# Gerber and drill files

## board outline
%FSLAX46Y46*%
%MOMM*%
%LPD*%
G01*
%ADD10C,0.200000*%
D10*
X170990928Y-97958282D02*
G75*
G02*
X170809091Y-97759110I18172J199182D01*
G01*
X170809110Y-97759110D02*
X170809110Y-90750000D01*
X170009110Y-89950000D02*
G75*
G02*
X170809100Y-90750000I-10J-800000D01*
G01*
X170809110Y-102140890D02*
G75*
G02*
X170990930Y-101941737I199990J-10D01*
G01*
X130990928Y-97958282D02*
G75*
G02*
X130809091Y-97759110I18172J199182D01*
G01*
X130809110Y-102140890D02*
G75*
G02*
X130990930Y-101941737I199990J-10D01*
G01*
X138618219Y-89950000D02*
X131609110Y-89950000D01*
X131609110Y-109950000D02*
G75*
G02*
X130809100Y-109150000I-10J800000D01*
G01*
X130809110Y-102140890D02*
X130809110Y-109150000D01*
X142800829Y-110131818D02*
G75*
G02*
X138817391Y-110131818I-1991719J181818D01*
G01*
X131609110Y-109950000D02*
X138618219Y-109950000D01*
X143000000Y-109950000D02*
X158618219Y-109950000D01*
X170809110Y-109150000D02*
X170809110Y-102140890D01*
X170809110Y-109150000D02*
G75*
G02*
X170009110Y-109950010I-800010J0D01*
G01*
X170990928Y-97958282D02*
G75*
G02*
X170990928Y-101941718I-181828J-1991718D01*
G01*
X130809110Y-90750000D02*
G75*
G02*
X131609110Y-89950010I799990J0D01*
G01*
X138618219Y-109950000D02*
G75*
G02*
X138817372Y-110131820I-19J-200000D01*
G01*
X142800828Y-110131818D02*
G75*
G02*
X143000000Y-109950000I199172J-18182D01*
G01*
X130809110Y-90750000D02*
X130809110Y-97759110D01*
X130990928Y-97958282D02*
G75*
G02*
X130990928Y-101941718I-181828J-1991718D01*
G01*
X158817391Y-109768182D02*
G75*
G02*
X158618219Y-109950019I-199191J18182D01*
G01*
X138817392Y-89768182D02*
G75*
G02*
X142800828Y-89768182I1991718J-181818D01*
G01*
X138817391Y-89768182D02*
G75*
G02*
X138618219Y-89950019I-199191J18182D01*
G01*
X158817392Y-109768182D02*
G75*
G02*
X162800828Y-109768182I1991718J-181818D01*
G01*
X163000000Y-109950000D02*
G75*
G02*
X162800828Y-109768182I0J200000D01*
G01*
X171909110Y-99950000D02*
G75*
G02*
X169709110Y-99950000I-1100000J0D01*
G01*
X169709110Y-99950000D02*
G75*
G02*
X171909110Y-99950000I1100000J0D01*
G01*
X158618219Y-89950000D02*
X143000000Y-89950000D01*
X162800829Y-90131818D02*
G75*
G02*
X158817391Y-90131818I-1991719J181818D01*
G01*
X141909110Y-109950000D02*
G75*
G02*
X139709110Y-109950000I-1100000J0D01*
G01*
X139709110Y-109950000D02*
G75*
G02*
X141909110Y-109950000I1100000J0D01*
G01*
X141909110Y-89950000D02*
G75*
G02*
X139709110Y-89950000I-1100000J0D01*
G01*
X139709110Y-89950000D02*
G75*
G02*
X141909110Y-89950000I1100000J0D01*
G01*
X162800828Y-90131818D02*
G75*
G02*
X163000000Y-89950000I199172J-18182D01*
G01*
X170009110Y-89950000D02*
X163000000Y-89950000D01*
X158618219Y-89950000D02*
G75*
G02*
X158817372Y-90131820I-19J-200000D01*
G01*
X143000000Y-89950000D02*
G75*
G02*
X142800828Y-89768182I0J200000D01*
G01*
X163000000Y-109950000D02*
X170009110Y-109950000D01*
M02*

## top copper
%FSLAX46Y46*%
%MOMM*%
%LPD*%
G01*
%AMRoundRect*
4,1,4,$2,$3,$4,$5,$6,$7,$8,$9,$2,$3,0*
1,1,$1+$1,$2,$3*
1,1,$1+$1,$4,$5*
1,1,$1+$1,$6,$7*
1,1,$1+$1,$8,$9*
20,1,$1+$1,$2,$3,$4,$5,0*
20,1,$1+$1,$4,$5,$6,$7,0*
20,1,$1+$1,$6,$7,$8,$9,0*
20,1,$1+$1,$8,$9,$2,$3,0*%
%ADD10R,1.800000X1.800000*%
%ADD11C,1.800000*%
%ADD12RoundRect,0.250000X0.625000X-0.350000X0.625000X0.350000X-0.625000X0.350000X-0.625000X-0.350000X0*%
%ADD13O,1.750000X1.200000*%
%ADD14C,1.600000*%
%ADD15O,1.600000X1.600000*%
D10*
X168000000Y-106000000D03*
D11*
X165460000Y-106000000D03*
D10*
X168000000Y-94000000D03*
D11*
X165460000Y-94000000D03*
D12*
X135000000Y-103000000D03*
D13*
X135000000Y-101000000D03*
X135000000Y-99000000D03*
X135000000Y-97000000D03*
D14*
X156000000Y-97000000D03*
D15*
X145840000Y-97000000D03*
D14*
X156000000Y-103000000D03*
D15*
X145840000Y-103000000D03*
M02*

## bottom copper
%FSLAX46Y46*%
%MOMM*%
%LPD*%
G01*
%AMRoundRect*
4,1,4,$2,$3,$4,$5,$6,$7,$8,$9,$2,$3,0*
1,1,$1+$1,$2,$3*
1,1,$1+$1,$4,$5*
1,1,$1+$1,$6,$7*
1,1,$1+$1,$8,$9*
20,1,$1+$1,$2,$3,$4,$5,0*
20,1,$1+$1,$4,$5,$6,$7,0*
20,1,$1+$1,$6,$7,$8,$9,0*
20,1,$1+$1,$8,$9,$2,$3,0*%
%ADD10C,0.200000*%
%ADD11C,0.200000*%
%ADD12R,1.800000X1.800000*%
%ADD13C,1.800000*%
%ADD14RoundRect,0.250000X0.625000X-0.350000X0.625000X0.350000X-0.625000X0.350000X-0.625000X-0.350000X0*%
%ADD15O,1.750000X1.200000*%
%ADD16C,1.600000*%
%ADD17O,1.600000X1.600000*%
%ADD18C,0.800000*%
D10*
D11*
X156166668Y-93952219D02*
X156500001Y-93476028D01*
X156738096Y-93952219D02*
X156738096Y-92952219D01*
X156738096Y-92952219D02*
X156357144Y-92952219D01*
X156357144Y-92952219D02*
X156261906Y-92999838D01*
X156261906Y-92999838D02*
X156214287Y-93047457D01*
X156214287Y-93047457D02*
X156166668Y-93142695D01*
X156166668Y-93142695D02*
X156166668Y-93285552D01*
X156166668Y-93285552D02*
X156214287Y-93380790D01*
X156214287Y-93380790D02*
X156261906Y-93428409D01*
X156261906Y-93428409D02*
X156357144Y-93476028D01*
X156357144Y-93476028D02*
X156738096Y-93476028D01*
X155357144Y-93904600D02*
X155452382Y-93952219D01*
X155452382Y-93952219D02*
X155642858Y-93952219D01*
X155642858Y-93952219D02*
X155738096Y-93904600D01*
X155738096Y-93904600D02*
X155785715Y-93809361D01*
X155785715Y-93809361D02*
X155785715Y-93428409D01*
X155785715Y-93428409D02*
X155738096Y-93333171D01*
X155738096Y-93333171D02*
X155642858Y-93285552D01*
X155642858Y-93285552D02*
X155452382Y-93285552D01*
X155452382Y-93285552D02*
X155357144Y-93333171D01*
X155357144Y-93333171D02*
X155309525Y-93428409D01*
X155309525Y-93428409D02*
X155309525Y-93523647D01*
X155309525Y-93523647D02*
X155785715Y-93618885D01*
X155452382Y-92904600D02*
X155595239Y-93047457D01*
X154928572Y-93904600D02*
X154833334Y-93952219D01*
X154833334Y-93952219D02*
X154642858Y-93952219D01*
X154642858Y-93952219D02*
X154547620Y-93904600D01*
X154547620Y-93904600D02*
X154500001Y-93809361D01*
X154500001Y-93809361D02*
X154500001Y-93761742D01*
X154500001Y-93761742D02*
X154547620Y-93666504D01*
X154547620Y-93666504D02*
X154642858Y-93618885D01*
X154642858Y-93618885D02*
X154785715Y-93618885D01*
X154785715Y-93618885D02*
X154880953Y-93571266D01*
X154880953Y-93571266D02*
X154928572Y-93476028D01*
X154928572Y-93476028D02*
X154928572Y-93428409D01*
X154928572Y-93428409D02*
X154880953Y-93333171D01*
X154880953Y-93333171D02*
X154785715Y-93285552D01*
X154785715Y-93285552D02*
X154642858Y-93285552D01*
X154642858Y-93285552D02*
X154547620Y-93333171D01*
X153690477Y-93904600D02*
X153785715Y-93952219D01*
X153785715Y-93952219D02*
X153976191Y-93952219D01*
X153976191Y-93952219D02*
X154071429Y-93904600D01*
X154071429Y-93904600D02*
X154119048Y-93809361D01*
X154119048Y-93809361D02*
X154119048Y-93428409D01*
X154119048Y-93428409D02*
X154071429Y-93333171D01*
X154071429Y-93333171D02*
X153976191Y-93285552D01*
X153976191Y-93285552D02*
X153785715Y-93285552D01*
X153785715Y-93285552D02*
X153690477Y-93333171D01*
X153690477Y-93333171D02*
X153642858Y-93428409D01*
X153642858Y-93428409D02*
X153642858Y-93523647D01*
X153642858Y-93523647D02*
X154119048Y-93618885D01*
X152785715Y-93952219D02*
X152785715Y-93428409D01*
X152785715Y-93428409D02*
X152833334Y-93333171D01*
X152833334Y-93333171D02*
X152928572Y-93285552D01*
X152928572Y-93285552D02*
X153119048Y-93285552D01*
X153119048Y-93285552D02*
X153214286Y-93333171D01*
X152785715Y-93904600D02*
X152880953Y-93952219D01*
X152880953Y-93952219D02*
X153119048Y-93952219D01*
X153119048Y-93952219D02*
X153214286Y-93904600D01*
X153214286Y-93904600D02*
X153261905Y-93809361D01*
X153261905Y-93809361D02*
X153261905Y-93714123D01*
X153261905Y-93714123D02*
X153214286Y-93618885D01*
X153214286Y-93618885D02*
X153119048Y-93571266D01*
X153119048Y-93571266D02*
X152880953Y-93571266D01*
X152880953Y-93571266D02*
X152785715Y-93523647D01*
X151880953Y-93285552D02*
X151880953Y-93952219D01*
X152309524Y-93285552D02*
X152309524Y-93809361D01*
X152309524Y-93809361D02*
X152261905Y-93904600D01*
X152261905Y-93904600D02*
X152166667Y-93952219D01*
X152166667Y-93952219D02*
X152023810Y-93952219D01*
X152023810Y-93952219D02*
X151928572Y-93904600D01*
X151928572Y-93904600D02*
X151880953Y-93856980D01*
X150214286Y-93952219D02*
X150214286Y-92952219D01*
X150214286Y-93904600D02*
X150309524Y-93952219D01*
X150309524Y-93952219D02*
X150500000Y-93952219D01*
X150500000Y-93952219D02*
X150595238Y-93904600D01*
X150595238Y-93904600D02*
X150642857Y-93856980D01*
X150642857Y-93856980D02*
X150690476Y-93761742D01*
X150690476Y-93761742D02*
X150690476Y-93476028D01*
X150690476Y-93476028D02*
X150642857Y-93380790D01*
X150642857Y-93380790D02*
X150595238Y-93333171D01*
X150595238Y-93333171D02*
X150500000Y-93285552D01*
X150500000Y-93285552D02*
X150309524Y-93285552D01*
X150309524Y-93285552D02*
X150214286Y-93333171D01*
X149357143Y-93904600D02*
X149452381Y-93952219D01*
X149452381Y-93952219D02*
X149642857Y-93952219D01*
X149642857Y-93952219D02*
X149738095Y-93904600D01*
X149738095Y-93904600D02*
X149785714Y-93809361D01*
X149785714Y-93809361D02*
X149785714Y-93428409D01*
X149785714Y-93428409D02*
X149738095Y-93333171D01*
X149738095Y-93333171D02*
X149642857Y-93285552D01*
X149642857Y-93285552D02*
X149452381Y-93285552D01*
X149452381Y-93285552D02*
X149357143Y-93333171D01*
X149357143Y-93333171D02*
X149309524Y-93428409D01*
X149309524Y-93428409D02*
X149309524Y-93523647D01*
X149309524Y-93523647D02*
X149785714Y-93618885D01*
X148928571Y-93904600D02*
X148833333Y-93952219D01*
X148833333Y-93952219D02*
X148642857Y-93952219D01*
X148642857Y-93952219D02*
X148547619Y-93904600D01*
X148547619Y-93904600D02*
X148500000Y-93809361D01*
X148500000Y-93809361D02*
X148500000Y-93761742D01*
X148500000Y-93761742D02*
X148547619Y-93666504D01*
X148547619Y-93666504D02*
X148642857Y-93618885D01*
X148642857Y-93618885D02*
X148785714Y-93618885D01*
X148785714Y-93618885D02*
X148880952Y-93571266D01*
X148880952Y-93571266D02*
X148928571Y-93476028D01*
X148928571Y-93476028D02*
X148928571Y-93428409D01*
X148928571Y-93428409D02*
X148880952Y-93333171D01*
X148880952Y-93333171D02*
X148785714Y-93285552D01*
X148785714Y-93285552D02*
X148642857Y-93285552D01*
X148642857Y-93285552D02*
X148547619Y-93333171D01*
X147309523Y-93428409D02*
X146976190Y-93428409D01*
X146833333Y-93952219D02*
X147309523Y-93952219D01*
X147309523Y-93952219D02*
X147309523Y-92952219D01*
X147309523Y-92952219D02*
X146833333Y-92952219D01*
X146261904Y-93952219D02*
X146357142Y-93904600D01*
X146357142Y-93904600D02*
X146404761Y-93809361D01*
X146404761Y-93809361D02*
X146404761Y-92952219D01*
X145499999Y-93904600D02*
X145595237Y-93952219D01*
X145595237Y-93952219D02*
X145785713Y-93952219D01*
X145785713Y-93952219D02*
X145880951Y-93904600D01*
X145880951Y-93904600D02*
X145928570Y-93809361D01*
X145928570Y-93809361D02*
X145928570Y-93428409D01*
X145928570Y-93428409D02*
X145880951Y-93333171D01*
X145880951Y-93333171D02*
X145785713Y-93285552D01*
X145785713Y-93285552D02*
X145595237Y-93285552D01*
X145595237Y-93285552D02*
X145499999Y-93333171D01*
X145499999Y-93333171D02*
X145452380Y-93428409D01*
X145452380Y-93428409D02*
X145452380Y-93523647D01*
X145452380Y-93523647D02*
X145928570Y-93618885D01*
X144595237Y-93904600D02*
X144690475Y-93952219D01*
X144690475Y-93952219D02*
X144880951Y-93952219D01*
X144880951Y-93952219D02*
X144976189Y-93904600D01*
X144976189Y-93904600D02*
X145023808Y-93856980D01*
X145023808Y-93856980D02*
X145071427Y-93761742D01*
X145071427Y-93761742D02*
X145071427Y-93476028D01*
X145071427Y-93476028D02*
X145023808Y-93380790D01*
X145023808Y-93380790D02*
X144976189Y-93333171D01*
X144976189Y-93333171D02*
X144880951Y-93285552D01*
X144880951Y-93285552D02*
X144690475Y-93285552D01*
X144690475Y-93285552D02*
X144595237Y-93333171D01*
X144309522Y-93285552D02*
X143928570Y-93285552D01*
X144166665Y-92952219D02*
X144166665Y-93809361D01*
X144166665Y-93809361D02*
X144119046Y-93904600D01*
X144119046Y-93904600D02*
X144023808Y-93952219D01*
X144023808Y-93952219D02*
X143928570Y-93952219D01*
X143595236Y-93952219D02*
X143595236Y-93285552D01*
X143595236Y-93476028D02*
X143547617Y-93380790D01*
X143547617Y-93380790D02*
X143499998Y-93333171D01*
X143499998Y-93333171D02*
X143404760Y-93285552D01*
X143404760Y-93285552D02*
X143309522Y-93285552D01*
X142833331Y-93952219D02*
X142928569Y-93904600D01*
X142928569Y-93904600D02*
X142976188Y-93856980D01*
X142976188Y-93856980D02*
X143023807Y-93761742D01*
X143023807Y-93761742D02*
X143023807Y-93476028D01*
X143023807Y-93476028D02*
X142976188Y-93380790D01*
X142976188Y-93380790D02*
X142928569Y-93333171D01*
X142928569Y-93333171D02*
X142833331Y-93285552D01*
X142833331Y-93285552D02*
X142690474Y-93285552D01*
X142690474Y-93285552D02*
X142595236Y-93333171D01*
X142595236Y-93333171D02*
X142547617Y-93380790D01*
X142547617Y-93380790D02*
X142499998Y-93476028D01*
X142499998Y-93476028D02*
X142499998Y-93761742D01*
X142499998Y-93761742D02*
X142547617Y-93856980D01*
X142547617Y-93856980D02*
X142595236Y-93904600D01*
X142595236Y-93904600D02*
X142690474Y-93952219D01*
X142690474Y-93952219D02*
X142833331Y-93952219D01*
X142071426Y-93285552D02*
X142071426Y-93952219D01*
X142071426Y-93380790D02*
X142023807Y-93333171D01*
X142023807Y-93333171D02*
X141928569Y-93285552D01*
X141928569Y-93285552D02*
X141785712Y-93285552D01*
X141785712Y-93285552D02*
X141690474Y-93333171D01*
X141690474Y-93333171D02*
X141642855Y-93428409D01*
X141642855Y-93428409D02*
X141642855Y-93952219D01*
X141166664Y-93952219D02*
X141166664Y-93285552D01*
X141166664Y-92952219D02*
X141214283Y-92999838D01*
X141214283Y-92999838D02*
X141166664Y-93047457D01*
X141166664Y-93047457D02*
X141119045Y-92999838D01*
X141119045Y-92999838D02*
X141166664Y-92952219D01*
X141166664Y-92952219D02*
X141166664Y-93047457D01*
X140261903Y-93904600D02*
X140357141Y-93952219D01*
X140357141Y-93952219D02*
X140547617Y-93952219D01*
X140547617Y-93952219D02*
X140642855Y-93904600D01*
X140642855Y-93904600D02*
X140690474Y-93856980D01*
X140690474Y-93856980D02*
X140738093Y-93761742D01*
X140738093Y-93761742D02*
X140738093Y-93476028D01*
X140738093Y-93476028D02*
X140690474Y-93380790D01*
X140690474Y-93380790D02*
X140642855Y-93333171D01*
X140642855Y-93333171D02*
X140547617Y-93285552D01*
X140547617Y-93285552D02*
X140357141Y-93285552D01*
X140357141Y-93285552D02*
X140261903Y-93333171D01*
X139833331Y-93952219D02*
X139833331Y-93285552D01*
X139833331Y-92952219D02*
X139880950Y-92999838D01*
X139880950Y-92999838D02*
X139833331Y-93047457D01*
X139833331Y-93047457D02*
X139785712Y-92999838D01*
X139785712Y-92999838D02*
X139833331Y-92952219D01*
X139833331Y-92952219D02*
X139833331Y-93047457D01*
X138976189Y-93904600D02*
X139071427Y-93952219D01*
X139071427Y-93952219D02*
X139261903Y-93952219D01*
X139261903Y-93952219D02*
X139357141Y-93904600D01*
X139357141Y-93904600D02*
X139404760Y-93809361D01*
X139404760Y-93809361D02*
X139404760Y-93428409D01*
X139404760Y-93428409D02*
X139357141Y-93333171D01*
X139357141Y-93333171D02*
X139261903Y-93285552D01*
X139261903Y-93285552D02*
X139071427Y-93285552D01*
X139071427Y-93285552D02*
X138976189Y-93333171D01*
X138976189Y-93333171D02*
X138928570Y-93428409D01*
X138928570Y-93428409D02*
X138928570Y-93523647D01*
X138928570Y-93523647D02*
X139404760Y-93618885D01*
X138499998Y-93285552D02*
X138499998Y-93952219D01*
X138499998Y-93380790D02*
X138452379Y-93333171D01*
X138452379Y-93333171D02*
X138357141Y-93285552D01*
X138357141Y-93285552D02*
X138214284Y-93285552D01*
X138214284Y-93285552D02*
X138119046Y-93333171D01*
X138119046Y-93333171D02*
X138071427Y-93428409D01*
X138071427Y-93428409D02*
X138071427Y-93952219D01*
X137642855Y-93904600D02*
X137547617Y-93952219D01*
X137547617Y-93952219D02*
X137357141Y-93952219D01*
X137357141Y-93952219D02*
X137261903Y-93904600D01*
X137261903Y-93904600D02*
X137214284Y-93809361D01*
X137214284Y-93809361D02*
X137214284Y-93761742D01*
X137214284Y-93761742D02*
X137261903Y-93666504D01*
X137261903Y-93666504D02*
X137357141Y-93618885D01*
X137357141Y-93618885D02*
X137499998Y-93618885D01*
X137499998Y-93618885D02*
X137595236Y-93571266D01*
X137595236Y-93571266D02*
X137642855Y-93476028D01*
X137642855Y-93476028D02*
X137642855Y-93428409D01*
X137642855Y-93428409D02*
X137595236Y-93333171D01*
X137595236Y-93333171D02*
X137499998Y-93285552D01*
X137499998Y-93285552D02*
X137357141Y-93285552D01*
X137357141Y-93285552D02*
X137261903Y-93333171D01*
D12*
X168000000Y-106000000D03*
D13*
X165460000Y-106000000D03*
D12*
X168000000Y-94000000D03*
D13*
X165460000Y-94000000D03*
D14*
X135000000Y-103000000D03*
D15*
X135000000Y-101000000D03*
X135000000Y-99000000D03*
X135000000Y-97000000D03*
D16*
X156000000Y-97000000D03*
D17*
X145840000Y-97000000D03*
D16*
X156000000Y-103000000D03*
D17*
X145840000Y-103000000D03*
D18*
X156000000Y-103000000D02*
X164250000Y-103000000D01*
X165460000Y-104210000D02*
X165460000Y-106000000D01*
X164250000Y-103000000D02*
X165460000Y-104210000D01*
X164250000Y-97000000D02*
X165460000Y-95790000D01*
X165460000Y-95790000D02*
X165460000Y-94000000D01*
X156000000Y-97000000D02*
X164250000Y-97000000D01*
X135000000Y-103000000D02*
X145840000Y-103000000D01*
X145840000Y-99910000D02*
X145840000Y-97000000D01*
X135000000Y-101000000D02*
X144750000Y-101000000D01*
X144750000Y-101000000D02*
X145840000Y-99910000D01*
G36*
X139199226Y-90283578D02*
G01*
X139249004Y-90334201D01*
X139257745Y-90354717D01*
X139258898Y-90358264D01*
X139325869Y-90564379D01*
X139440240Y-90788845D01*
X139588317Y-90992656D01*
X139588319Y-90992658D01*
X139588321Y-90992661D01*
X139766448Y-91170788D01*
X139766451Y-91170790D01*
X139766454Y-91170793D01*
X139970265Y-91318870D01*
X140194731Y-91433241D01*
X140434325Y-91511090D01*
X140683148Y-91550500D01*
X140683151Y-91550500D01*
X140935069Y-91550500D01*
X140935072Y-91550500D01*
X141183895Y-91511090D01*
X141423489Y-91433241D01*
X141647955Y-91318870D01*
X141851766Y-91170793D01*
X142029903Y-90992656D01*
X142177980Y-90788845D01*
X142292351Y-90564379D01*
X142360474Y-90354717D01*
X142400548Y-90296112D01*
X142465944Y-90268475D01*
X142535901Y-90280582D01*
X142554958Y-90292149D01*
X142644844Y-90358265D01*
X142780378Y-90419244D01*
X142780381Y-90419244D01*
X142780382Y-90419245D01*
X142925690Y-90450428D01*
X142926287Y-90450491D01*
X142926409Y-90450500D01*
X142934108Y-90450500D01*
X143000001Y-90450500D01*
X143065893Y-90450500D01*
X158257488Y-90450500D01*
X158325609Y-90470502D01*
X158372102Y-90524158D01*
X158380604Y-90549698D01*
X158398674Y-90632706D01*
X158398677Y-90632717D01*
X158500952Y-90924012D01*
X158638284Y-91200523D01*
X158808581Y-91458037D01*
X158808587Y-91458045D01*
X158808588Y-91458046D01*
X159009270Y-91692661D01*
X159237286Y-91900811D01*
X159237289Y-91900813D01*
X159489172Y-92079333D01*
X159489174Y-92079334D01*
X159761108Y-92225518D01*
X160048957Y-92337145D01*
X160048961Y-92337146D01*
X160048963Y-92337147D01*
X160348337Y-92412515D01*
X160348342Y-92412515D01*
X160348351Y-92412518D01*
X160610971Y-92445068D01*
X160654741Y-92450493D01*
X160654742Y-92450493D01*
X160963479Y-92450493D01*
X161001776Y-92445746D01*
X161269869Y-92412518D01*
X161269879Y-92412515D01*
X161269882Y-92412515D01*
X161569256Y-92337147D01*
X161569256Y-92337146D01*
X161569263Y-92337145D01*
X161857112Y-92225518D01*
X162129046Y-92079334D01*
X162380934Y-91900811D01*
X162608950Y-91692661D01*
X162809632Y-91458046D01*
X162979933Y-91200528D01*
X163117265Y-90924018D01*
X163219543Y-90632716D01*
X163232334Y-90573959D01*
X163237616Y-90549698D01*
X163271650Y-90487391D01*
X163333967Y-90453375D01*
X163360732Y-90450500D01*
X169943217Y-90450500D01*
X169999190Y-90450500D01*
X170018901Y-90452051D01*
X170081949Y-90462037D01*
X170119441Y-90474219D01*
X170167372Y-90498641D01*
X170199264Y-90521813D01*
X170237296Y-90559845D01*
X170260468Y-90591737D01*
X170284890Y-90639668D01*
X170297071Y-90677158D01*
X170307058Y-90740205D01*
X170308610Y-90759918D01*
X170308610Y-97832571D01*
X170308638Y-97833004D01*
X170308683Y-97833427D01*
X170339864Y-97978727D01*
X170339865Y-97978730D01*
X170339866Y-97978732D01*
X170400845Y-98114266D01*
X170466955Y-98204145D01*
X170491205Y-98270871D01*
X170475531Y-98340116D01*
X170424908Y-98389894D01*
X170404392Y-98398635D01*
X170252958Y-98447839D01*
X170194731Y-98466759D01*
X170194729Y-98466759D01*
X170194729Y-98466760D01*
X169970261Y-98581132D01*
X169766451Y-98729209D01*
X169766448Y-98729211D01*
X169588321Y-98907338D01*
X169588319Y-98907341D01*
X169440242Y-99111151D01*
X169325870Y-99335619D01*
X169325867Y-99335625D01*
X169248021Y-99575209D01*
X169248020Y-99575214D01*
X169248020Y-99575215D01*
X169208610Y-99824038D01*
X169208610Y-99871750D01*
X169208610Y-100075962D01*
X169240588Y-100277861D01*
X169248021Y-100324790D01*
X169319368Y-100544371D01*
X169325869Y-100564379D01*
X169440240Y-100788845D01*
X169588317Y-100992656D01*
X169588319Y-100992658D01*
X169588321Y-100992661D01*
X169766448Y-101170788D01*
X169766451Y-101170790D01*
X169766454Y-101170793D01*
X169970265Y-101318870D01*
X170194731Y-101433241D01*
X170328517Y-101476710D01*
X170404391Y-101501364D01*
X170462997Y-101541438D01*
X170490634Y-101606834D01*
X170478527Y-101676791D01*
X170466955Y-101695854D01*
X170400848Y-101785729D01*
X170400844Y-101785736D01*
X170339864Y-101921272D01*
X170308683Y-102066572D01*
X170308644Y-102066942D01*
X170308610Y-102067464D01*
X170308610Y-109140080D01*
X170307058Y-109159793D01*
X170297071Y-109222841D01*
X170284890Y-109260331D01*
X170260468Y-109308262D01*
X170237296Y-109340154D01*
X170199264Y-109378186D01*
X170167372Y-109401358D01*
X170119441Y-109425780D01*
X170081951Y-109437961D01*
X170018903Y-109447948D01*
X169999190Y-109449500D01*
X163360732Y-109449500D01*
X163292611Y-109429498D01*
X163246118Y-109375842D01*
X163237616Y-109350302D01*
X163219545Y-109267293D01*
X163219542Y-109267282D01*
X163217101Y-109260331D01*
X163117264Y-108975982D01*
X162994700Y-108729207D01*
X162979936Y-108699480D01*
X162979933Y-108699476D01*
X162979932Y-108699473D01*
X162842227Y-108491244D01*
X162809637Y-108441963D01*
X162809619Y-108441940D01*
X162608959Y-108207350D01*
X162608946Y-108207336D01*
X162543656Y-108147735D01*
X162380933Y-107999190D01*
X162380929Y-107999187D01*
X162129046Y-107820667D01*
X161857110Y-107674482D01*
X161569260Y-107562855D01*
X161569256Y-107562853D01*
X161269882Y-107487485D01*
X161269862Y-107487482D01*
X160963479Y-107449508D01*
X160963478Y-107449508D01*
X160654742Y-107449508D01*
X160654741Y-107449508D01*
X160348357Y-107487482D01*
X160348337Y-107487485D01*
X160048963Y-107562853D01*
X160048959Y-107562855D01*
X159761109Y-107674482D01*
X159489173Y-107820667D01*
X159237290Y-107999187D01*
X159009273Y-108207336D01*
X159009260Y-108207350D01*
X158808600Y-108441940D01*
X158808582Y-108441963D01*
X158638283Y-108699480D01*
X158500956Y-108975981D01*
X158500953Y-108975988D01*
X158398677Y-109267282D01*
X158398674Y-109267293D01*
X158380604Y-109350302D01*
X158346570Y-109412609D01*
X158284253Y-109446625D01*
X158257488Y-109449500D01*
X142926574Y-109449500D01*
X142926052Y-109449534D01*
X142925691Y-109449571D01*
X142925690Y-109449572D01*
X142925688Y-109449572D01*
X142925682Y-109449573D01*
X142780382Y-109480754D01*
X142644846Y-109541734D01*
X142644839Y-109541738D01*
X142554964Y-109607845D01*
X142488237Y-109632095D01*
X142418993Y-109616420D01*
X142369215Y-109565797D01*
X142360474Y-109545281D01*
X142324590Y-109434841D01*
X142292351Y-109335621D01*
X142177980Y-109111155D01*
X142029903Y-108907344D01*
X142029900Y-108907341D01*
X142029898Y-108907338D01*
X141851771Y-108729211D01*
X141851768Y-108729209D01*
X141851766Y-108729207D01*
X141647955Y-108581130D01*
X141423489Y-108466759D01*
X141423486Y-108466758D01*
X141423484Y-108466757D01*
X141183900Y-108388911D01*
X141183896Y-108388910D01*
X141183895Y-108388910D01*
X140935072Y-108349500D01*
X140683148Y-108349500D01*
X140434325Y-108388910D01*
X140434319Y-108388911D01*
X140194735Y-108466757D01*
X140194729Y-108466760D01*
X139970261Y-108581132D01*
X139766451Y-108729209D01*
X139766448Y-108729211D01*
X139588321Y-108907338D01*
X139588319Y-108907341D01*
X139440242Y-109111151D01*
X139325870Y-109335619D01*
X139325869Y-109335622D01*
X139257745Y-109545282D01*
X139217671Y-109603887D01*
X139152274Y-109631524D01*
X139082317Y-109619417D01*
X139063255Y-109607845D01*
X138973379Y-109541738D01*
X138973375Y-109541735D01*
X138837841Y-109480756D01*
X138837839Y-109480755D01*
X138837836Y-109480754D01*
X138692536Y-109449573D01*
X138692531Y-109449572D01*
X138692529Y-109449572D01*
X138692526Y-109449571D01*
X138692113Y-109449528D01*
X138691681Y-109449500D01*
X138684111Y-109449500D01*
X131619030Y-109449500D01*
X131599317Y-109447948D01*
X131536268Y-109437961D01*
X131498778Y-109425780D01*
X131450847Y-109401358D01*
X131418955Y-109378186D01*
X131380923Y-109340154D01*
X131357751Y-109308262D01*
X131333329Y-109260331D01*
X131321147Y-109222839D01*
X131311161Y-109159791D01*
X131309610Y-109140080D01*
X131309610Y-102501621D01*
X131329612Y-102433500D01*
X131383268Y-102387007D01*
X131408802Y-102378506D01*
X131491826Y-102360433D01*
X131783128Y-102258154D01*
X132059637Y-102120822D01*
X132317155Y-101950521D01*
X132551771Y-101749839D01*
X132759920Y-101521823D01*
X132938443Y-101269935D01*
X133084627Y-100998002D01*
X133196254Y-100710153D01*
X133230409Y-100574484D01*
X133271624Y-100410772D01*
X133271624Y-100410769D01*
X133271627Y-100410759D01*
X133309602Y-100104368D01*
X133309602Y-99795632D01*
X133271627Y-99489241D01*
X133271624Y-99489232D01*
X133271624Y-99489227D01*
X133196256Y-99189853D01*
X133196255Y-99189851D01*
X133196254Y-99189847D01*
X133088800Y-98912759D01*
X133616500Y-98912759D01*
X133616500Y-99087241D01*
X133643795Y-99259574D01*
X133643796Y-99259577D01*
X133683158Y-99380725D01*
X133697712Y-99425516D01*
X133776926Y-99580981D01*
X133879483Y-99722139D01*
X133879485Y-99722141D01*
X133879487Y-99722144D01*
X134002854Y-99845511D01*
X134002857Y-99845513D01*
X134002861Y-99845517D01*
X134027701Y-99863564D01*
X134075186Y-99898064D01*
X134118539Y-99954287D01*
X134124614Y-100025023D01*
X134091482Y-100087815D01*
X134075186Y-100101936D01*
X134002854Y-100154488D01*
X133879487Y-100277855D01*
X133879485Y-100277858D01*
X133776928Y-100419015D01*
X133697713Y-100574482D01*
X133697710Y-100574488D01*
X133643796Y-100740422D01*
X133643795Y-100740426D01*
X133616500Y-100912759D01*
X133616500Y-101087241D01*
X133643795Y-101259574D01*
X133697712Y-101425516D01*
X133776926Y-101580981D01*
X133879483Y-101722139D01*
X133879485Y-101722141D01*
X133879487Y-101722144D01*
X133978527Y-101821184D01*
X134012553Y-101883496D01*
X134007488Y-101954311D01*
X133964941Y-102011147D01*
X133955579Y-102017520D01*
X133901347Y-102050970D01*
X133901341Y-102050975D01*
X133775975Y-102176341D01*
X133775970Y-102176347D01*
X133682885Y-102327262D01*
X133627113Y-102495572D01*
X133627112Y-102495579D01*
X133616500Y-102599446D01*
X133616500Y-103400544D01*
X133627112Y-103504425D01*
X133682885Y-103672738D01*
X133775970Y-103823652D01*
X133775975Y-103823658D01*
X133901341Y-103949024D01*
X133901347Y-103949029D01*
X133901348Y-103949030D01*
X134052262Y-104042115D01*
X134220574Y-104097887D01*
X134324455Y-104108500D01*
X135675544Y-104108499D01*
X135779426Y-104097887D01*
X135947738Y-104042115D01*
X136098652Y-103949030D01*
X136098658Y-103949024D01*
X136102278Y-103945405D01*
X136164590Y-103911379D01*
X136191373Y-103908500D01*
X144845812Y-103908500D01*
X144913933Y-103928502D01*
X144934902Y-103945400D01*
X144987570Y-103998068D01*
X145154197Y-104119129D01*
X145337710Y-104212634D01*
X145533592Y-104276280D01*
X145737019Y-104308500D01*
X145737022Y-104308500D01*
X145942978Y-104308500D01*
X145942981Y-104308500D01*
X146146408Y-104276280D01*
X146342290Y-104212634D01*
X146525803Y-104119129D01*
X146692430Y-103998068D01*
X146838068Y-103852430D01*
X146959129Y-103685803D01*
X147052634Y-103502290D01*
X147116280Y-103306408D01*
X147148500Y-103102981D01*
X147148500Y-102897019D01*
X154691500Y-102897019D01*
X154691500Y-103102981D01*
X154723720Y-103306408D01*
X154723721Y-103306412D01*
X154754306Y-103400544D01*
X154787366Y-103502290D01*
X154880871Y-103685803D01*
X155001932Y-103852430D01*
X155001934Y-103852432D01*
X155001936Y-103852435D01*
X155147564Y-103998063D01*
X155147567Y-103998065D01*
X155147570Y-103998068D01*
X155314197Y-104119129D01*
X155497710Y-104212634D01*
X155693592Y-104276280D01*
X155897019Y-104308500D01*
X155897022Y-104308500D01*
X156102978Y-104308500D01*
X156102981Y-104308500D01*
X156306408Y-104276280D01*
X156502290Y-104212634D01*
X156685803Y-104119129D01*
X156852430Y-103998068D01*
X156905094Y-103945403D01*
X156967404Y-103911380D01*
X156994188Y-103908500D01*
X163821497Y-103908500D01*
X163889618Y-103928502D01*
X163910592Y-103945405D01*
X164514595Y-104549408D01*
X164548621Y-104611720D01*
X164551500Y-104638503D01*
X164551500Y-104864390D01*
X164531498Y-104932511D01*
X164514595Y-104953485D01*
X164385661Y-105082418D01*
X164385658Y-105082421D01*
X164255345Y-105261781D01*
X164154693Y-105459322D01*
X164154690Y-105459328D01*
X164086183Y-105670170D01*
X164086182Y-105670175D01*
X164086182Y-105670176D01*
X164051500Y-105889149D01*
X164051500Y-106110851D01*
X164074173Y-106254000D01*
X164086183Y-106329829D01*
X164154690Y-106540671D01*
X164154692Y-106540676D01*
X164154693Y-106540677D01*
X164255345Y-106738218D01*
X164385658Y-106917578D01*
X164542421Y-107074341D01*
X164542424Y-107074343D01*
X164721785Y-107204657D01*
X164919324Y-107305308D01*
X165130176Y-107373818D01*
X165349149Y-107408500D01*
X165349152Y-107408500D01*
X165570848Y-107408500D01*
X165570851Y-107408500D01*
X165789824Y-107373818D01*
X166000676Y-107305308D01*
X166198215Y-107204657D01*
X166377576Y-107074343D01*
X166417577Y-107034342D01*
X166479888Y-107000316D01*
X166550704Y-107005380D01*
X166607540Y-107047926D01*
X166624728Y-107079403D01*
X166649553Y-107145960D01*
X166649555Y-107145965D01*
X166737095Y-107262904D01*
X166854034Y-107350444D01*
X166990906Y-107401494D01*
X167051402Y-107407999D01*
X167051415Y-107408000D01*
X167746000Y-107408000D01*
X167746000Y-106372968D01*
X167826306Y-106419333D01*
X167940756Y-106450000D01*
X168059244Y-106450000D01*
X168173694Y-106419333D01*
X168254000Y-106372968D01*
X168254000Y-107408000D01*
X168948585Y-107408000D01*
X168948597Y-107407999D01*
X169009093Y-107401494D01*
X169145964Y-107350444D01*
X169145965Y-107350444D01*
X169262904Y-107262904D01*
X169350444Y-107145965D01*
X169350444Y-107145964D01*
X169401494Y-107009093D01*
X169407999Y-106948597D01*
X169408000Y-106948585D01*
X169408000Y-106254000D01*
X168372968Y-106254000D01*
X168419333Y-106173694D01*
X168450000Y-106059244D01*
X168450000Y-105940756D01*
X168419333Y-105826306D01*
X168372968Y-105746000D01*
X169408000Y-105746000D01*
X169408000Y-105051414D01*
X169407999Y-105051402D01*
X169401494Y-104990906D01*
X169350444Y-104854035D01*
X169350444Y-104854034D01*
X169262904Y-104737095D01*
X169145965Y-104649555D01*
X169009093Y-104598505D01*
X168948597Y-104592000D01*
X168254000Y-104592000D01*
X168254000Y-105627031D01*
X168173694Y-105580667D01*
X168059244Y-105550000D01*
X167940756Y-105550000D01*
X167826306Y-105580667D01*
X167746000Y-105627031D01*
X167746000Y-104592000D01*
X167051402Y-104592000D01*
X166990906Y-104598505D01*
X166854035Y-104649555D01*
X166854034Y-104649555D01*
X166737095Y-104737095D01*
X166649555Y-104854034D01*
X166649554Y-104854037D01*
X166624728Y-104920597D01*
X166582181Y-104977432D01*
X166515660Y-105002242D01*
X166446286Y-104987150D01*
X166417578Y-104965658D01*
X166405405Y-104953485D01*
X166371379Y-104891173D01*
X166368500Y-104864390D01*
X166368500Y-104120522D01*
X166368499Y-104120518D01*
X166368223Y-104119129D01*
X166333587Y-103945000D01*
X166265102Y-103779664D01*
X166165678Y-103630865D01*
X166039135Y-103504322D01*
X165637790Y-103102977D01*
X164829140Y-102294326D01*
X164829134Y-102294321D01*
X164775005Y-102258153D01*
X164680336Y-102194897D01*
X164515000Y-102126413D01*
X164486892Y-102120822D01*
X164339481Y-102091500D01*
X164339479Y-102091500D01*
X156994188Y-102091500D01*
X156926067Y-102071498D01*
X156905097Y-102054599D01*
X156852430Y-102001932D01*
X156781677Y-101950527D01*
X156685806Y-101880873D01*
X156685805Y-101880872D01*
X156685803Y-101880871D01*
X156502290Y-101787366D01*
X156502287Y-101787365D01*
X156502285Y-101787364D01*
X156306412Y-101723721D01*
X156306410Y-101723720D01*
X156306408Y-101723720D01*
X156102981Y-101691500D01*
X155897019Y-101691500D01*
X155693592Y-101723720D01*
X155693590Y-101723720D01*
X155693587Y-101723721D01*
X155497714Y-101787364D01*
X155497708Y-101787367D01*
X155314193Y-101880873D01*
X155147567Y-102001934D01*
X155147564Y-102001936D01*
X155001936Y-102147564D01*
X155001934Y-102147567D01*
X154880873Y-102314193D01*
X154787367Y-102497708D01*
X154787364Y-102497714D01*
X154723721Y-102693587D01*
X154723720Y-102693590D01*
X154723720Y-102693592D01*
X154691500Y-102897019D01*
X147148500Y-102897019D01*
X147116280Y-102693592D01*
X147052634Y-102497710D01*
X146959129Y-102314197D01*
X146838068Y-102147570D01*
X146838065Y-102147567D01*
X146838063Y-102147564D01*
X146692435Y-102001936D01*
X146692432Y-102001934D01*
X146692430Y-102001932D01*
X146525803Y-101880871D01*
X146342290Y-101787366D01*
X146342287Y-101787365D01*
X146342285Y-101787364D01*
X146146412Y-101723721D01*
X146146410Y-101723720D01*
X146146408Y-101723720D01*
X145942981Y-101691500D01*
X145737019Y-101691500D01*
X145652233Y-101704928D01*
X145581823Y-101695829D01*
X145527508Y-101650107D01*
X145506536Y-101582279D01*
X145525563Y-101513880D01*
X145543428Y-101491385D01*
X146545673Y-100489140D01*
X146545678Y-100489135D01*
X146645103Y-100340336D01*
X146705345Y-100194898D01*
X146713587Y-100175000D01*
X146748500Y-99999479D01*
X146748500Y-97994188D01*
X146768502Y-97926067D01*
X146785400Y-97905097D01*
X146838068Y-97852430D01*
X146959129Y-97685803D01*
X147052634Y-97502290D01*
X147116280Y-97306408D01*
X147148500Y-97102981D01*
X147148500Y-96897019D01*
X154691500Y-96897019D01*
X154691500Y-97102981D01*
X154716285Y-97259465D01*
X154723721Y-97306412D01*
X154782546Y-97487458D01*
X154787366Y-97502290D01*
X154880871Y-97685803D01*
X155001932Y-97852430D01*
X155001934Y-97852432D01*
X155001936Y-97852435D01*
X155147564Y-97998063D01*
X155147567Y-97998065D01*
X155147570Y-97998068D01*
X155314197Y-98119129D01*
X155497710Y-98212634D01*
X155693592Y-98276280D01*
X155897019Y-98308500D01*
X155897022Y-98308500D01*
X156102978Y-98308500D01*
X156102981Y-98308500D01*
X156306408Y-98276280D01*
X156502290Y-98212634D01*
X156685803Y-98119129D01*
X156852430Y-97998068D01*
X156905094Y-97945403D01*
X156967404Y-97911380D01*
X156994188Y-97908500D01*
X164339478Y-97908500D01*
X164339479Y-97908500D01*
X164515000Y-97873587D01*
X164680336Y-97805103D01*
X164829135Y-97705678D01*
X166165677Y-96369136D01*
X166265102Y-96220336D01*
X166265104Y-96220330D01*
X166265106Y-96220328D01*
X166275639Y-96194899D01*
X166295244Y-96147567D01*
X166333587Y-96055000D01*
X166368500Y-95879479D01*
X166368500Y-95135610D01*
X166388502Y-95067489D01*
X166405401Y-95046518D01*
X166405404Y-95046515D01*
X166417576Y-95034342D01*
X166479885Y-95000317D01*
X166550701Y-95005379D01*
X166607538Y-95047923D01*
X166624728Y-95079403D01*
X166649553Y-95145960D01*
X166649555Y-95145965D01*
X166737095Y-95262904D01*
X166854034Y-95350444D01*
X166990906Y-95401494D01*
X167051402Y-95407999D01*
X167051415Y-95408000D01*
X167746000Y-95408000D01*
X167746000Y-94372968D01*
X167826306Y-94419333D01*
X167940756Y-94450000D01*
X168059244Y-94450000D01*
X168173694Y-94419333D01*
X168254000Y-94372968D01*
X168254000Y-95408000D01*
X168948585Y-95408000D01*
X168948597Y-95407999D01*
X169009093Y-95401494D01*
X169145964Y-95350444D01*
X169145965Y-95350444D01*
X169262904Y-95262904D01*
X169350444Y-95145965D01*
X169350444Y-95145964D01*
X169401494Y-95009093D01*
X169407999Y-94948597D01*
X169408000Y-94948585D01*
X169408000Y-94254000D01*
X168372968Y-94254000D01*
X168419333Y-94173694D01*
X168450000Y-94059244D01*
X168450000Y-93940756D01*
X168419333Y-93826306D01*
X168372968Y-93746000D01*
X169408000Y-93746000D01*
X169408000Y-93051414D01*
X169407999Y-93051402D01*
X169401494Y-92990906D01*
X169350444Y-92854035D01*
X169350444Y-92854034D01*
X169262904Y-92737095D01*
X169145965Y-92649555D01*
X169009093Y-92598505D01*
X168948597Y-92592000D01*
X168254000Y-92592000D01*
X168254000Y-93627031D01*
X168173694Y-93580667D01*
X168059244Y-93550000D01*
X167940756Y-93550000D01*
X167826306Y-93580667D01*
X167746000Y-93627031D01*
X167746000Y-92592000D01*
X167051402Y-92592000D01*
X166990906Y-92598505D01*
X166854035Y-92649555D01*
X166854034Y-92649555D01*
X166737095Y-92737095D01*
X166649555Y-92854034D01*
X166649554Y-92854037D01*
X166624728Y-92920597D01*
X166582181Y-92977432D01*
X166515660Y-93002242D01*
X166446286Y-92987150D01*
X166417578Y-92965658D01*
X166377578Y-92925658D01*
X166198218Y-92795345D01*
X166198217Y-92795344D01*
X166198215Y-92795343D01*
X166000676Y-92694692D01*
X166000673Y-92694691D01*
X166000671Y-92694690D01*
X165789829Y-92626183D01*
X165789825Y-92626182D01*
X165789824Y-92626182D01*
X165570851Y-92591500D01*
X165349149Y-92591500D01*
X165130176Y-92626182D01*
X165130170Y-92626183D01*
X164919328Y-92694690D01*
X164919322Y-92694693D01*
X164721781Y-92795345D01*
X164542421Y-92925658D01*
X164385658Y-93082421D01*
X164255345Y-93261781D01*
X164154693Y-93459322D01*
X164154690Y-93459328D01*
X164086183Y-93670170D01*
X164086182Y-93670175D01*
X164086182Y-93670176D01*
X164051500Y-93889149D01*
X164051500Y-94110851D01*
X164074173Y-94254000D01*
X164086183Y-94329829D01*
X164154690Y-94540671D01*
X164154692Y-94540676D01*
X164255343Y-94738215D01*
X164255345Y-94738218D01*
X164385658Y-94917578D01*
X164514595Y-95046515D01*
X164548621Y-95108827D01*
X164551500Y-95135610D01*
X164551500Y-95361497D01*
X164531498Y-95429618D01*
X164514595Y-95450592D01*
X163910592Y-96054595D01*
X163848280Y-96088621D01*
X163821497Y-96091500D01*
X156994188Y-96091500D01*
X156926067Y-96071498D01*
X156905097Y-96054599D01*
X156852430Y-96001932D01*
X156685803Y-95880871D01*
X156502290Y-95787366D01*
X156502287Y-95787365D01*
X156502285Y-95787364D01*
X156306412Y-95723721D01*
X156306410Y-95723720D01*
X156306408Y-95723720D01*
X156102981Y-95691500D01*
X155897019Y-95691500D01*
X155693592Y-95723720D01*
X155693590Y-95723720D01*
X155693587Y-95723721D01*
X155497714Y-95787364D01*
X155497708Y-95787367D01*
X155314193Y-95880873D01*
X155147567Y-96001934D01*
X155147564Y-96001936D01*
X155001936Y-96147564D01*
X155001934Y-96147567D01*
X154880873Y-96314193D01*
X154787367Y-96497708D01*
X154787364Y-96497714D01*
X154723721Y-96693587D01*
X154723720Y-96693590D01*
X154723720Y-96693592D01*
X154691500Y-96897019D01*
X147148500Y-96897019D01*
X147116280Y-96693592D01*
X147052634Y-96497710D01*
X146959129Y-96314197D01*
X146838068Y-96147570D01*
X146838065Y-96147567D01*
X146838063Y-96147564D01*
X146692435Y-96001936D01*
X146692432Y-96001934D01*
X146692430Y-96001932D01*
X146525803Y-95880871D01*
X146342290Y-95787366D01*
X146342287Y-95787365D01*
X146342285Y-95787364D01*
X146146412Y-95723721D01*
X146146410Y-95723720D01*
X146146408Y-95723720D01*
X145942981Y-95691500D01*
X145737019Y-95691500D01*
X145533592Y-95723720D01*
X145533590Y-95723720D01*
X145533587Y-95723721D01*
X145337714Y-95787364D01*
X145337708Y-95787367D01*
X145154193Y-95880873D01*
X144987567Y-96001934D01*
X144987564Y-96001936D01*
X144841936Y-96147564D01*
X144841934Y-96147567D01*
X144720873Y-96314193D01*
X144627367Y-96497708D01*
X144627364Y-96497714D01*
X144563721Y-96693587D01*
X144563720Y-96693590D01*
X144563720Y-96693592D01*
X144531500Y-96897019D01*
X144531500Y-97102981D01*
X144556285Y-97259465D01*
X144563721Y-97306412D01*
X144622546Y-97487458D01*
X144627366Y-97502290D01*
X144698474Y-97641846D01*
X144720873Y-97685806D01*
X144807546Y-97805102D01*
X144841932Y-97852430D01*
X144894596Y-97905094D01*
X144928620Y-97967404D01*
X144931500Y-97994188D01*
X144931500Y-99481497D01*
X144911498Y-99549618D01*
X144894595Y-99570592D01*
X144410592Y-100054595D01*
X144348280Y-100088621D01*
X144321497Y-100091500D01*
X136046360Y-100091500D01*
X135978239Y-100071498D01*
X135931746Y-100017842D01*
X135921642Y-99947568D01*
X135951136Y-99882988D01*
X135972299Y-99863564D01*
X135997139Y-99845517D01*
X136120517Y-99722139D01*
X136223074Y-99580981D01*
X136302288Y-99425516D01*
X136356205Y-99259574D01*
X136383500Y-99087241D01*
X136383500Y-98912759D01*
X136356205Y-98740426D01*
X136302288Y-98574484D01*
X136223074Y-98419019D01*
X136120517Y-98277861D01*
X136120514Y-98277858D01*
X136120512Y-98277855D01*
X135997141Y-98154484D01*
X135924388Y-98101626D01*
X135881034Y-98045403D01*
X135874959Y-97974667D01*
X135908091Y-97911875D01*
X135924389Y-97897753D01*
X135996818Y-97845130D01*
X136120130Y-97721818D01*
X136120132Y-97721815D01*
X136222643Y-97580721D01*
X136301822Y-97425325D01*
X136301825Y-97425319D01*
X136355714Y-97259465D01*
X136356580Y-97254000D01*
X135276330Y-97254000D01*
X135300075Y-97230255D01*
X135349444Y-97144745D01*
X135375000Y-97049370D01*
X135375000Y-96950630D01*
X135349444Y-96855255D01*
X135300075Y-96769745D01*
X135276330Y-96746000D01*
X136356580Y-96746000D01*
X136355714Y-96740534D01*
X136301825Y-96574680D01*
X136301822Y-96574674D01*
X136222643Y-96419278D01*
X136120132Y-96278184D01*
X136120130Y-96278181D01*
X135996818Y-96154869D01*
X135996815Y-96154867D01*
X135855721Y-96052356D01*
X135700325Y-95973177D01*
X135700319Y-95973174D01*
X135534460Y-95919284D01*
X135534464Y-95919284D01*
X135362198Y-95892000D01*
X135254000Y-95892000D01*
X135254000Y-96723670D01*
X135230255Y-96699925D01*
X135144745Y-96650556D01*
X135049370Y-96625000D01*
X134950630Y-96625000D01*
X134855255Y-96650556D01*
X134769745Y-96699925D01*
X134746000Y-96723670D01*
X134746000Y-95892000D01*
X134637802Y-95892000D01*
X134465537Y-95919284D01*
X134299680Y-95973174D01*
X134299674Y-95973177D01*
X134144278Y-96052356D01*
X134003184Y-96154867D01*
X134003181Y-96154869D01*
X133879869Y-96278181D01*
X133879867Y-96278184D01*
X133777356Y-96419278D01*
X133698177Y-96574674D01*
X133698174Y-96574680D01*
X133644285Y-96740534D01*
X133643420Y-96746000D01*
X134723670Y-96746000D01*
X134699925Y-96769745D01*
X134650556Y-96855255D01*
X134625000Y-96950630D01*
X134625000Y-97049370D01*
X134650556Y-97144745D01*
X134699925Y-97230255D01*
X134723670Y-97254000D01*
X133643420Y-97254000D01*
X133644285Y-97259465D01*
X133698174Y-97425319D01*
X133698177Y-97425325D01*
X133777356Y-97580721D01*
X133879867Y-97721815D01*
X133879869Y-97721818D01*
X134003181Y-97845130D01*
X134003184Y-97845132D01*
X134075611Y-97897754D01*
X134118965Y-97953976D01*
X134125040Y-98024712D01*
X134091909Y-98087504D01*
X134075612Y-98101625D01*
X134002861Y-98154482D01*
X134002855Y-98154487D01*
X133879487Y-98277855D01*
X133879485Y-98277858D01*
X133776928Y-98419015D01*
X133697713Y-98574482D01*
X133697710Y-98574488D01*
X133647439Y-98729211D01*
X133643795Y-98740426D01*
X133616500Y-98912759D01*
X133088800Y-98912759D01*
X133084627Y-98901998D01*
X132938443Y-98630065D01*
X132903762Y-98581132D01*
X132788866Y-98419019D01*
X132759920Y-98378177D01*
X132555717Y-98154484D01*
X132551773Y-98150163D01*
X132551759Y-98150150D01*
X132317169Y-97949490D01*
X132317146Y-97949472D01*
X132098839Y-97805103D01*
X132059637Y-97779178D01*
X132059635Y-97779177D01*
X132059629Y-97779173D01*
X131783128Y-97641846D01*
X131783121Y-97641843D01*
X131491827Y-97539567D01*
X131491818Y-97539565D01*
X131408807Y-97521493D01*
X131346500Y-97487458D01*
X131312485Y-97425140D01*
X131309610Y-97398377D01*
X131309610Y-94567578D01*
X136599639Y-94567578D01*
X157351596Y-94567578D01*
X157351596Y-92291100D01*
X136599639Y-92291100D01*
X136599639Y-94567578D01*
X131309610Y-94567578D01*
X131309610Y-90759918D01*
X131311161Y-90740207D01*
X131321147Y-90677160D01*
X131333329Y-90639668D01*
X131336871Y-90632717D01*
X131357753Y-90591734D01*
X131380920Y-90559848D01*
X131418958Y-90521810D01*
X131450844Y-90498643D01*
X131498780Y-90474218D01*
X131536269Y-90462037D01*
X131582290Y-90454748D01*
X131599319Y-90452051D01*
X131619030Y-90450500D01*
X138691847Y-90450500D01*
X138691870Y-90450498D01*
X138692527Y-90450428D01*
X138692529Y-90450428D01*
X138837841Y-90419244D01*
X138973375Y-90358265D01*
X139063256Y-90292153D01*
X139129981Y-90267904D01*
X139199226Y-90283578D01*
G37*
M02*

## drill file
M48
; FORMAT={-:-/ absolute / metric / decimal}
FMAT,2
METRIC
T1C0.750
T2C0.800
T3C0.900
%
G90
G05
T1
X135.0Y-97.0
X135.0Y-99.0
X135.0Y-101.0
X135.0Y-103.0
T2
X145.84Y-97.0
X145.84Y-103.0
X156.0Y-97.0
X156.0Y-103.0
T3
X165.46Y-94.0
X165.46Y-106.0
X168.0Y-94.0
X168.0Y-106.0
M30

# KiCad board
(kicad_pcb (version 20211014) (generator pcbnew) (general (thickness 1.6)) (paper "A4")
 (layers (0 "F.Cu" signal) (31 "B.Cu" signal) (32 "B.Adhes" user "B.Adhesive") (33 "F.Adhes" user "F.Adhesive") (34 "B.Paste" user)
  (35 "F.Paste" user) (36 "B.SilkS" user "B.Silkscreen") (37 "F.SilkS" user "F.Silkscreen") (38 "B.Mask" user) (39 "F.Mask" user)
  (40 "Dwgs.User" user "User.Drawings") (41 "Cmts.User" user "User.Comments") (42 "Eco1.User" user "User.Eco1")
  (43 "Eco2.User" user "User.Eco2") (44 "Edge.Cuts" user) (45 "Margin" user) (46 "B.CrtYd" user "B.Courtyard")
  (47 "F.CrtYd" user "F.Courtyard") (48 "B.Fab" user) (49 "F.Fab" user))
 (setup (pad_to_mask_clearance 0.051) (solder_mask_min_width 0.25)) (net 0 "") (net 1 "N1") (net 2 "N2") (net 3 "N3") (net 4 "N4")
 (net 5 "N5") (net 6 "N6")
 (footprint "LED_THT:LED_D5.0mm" (layer "F.Cu") (at 168 106 180)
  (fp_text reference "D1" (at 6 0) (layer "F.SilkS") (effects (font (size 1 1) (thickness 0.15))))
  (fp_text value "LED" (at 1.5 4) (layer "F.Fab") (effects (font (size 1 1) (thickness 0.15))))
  (pad "1" thru_hole rect (at 0 0 180) (size 1.8 1.8) (drill 0.9) (layers *.Cu *.Mask) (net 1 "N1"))
  (pad "2" thru_hole circle (at 2.54 0 180) (size 1.8 1.8) (drill 0.9) (layers *.Cu *.Mask) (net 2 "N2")))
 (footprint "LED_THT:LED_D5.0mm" (layer "F.Cu") (at 168 94 180)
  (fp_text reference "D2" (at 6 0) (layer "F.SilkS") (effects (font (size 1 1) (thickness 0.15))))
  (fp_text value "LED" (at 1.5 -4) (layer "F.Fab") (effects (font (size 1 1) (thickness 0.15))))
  (pad "1" thru_hole rect (at 0 0 180) (size 1.8 1.8) (drill 0.9) (layers *.Cu *.Mask) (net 1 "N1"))
  (pad "2" thru_hole circle (at 2.54 0 180) (size 1.8 1.8) (drill 0.9) (layers *.Cu *.Mask) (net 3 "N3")))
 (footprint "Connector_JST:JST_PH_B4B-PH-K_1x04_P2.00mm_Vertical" (layer "F.Cu") (at 135 103 90)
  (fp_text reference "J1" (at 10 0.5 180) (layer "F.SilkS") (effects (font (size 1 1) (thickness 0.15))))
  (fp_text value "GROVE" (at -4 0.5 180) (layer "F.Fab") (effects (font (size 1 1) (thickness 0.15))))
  (pad "1" thru_hole roundrect (at 0 0 90) (size 1.2 1.75) (drill 0.75) (layers *.Cu *.Mask) (roundrect_rratio 0.208333) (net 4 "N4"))
  (pad "2" thru_hole oval (at 2 0 90) (size 1.2 1.75) (drill 0.75) (layers *.Cu *.Mask) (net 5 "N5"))
  (pad "3" thru_hole oval (at 4 0 90) (size 1.2 1.75) (drill 0.75) (layers *.Cu *.Mask) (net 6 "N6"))
  (pad "4" thru_hole oval (at 6 0 90) (size 1.2 1.75) (drill 0.75) (layers *.Cu *.Mask) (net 1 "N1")))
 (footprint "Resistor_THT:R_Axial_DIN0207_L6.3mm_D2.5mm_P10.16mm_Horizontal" (layer "F.Cu") (at 156 97 180)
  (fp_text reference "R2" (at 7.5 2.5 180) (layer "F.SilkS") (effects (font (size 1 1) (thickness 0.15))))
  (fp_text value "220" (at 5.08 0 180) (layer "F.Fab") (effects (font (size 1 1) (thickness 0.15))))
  (pad "1" thru_hole circle (at 0 0 180) (size 1.6 1.6) (drill 0.8) (layers *.Cu *.Mask) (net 3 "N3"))
  (pad "2" thru_hole oval (at 10.16 0 180) (size 1.6 1.6) (drill 0.8) (layers *.Cu *.Mask) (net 5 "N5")))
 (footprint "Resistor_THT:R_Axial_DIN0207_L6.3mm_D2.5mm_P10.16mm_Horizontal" (layer "F.Cu") (at 156 103 180)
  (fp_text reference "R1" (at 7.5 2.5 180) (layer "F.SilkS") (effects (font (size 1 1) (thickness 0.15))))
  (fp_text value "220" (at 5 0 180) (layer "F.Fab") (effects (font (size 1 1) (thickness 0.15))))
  (pad "1" thru_hole circle (at 0 0 180) (size 1.6 1.6) (drill 0.8) (layers *.Cu *.Mask) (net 2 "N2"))
  (pad "2" thru_hole oval (at 10.16 0 180) (size 1.6 1.6) (drill 0.8) (layers *.Cu *.Mask) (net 4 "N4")))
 (gr_arc (start 170.990928 97.958282) (mid 170.8614 97.89395) (end 170.80911 97.75911) (layer "Edge.Cuts") (width 0.2))
 (gr_line (start 170.80911 97.75911) (end 170.80911 90.75) (layer "Edge.Cuts") (width 0.2))
 (gr_arc (start 170.00911 89.95) (mid 170.574795 90.184315) (end 170.80911 90.75) (layer "Edge.Cuts") (width 0.2))
 (gr_arc (start 170.80911 102.14089) (mid 170.8614 102.00605) (end 170.990928 101.941718) (layer "Edge.Cuts") (width 0.2))
 (gr_arc (start 130.990928 97.958282) (mid 130.8614 97.89395) (end 130.80911 97.75911) (layer "Edge.Cuts") (width 0.2))
 (gr_arc (start 130.80911 102.14089) (mid 130.8614 102.00605) (end 130.990928 101.941718) (layer "Edge.Cuts") (width 0.2))
 (gr_line (start 138.618219 89.95) (end 131.60911 89.95) (layer "Edge.Cuts") (width 0.2))
 (gr_arc (start 131.60911 109.95) (mid 131.043425 109.715685) (end 130.80911 109.15) (layer "Edge.Cuts") (width 0.2))
 (gr_line (start 130.80911 102.14089) (end 130.80911 109.15) (layer "Edge.Cuts") (width 0.2))
 (gr_arc (start 142.800829 110.131818) (mid 140.80911 111.950001) (end 138.817391 110.131818) (layer "Edge.Cuts") (width 0.2))
 (gr_line (start 131.60911 109.95) (end 138.618219 109.95) (layer "Edge.Cuts") (width 0.2))
 (gr_line (start 143 109.95) (end 158.618219 109.95) (layer "Edge.Cuts") (width 0.2))
 (gr_line (start 170.80911 109.15) (end 170.80911 102.14089) (layer "Edge.Cuts") (width 0.2))
 (gr_arc (start 170.80911 109.15) (mid 170.574795 109.715685) (end 170.00911 109.95) (layer "Edge.Cuts") (width 0.2))
 (gr_arc (start 170.990928 97.958282) (mid 172.80911 99.95) (end 170.990928 101.941718) (layer "Edge.Cuts") (width 0.2))
 (gr_arc (start 130.80911 90.75) (mid 131.043425 90.184315) (end 131.60911 89.95) (layer "Edge.Cuts") (width 0.2))
 (gr_arc (start 138.618219 109.95) (mid 138.753059 110.00229) (end 138.817391 110.131818) (layer "Edge.Cuts") (width 0.2))
 (gr_arc (start 142.800828 110.131818) (mid 142.86516 110.00229) (end 143 109.95) (layer "Edge.Cuts") (width 0.2))
 (gr_line (start 130.80911 90.75) (end 130.80911 97.75911) (layer "Edge.Cuts") (width 0.2))
 (gr_arc (start 130.990928 97.958282) (mid 132.80911 99.95) (end 130.990928 101.941718) (layer "Edge.Cuts") (width 0.2))
 (gr_arc (start 158.817391 109.768182) (mid 158.753059 109.89771) (end 158.618219 109.95) (layer "Edge.Cuts") (width 0.2))
 (gr_arc (start 138.817392 89.768182) (mid 140.80911 87.95) (end 142.800828 89.768182) (layer "Edge.Cuts") (width 0.2))
 (gr_arc (start 138.817391 89.768182) (mid 138.753059 89.89771) (end 138.618219 89.95) (layer "Edge.Cuts") (width 0.2))
 (gr_arc (start 158.817392 109.768182) (mid 160.80911 107.95) (end 162.800828 109.768182) (layer "Edge.Cuts") (width 0.2))
 (gr_arc (start 163 109.95) (mid 162.86516 109.89771) (end 162.800828 109.768182) (layer "Edge.Cuts") (width 0.2))
 (gr_circle (center 170.80911 99.95) (end 171.90911 99.95) (layer "Edge.Cuts") (width 0.2) (fill none))
 (gr_line (start 158.618219 89.95) (end 143 89.95) (layer "Edge.Cuts") (width 0.2))
 (gr_arc (start 162.800829 90.131818) (mid 160.80911 91.950001) (end 158.817391 90.131818) (layer "Edge.Cuts") (width 0.2))
 (gr_circle (center 140.80911 109.95) (end 141.90911 109.95) (layer "Edge.Cuts") (width 0.2) (fill none))
 (gr_circle (center 140.80911 89.95) (end 141.90911 89.95) (layer "Edge.Cuts") (width 0.2) (fill none))
 (gr_arc (start 162.800828 90.131818) (mid 162.86516 90.00229) (end 163 89.95) (layer "Edge.Cuts") (width 0.2))
 (gr_line (start 170.00911 89.95) (end 163 89.95) (layer "Edge.Cuts") (width 0.2))
 (gr_arc (start 158.618219 89.95) (mid 158.753059 90.00229) (end 158.817391 90.131818) (layer "Edge.Cuts") (width 0.2))
 (gr_arc (start 143 89.95) (mid 142.86516 89.89771) (end 142.800828 89.768182) (layer "Edge.Cuts") (width 0.2))
 (gr_line (start 163 109.95) (end 170.00911 109.95) (layer "Edge.Cuts") (width 0.2))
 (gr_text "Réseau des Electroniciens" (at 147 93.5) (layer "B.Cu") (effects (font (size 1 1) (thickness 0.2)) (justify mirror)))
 (segment (start 156 103) (end 164.25 103) (width 0.8) (layer "B.Cu") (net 2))
 (segment (start 165.46 104.21) (end 165.46 106) (width 0.8) (layer "B.Cu") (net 2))
 (segment (start 164.25 103) (end 165.46 104.21) (width 0.8) (layer "B.Cu") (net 2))
 (segment (start 164.25 97) (end 165.46 95.79) (width 0.8) (layer "B.Cu") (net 3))
 (segment (start 165.46 95.79) (end 165.46 94) (width 0.8) (layer "B.Cu") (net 3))
 (segment (start 156 97) (end 164.25 97) (width 0.8) (layer "B.Cu") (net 3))
 (segment (start 135 103) (end 145.84 103) (width 0.8) (layer "B.Cu") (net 4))
 (segment (start 145.84 99.91) (end 145.84 97) (width 0.8) (layer "B.Cu") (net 5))
 (segment (start 135 101) (end 144.75 101) (width 0.8) (layer "B.Cu") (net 5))
 (segment (start 144.75 101) (end 145.84 99.91) (width 0.8) (layer "B.Cu") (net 5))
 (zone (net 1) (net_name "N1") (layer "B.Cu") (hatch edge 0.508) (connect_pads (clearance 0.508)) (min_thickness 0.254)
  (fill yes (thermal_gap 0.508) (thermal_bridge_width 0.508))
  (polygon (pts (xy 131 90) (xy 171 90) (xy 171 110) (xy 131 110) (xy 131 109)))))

